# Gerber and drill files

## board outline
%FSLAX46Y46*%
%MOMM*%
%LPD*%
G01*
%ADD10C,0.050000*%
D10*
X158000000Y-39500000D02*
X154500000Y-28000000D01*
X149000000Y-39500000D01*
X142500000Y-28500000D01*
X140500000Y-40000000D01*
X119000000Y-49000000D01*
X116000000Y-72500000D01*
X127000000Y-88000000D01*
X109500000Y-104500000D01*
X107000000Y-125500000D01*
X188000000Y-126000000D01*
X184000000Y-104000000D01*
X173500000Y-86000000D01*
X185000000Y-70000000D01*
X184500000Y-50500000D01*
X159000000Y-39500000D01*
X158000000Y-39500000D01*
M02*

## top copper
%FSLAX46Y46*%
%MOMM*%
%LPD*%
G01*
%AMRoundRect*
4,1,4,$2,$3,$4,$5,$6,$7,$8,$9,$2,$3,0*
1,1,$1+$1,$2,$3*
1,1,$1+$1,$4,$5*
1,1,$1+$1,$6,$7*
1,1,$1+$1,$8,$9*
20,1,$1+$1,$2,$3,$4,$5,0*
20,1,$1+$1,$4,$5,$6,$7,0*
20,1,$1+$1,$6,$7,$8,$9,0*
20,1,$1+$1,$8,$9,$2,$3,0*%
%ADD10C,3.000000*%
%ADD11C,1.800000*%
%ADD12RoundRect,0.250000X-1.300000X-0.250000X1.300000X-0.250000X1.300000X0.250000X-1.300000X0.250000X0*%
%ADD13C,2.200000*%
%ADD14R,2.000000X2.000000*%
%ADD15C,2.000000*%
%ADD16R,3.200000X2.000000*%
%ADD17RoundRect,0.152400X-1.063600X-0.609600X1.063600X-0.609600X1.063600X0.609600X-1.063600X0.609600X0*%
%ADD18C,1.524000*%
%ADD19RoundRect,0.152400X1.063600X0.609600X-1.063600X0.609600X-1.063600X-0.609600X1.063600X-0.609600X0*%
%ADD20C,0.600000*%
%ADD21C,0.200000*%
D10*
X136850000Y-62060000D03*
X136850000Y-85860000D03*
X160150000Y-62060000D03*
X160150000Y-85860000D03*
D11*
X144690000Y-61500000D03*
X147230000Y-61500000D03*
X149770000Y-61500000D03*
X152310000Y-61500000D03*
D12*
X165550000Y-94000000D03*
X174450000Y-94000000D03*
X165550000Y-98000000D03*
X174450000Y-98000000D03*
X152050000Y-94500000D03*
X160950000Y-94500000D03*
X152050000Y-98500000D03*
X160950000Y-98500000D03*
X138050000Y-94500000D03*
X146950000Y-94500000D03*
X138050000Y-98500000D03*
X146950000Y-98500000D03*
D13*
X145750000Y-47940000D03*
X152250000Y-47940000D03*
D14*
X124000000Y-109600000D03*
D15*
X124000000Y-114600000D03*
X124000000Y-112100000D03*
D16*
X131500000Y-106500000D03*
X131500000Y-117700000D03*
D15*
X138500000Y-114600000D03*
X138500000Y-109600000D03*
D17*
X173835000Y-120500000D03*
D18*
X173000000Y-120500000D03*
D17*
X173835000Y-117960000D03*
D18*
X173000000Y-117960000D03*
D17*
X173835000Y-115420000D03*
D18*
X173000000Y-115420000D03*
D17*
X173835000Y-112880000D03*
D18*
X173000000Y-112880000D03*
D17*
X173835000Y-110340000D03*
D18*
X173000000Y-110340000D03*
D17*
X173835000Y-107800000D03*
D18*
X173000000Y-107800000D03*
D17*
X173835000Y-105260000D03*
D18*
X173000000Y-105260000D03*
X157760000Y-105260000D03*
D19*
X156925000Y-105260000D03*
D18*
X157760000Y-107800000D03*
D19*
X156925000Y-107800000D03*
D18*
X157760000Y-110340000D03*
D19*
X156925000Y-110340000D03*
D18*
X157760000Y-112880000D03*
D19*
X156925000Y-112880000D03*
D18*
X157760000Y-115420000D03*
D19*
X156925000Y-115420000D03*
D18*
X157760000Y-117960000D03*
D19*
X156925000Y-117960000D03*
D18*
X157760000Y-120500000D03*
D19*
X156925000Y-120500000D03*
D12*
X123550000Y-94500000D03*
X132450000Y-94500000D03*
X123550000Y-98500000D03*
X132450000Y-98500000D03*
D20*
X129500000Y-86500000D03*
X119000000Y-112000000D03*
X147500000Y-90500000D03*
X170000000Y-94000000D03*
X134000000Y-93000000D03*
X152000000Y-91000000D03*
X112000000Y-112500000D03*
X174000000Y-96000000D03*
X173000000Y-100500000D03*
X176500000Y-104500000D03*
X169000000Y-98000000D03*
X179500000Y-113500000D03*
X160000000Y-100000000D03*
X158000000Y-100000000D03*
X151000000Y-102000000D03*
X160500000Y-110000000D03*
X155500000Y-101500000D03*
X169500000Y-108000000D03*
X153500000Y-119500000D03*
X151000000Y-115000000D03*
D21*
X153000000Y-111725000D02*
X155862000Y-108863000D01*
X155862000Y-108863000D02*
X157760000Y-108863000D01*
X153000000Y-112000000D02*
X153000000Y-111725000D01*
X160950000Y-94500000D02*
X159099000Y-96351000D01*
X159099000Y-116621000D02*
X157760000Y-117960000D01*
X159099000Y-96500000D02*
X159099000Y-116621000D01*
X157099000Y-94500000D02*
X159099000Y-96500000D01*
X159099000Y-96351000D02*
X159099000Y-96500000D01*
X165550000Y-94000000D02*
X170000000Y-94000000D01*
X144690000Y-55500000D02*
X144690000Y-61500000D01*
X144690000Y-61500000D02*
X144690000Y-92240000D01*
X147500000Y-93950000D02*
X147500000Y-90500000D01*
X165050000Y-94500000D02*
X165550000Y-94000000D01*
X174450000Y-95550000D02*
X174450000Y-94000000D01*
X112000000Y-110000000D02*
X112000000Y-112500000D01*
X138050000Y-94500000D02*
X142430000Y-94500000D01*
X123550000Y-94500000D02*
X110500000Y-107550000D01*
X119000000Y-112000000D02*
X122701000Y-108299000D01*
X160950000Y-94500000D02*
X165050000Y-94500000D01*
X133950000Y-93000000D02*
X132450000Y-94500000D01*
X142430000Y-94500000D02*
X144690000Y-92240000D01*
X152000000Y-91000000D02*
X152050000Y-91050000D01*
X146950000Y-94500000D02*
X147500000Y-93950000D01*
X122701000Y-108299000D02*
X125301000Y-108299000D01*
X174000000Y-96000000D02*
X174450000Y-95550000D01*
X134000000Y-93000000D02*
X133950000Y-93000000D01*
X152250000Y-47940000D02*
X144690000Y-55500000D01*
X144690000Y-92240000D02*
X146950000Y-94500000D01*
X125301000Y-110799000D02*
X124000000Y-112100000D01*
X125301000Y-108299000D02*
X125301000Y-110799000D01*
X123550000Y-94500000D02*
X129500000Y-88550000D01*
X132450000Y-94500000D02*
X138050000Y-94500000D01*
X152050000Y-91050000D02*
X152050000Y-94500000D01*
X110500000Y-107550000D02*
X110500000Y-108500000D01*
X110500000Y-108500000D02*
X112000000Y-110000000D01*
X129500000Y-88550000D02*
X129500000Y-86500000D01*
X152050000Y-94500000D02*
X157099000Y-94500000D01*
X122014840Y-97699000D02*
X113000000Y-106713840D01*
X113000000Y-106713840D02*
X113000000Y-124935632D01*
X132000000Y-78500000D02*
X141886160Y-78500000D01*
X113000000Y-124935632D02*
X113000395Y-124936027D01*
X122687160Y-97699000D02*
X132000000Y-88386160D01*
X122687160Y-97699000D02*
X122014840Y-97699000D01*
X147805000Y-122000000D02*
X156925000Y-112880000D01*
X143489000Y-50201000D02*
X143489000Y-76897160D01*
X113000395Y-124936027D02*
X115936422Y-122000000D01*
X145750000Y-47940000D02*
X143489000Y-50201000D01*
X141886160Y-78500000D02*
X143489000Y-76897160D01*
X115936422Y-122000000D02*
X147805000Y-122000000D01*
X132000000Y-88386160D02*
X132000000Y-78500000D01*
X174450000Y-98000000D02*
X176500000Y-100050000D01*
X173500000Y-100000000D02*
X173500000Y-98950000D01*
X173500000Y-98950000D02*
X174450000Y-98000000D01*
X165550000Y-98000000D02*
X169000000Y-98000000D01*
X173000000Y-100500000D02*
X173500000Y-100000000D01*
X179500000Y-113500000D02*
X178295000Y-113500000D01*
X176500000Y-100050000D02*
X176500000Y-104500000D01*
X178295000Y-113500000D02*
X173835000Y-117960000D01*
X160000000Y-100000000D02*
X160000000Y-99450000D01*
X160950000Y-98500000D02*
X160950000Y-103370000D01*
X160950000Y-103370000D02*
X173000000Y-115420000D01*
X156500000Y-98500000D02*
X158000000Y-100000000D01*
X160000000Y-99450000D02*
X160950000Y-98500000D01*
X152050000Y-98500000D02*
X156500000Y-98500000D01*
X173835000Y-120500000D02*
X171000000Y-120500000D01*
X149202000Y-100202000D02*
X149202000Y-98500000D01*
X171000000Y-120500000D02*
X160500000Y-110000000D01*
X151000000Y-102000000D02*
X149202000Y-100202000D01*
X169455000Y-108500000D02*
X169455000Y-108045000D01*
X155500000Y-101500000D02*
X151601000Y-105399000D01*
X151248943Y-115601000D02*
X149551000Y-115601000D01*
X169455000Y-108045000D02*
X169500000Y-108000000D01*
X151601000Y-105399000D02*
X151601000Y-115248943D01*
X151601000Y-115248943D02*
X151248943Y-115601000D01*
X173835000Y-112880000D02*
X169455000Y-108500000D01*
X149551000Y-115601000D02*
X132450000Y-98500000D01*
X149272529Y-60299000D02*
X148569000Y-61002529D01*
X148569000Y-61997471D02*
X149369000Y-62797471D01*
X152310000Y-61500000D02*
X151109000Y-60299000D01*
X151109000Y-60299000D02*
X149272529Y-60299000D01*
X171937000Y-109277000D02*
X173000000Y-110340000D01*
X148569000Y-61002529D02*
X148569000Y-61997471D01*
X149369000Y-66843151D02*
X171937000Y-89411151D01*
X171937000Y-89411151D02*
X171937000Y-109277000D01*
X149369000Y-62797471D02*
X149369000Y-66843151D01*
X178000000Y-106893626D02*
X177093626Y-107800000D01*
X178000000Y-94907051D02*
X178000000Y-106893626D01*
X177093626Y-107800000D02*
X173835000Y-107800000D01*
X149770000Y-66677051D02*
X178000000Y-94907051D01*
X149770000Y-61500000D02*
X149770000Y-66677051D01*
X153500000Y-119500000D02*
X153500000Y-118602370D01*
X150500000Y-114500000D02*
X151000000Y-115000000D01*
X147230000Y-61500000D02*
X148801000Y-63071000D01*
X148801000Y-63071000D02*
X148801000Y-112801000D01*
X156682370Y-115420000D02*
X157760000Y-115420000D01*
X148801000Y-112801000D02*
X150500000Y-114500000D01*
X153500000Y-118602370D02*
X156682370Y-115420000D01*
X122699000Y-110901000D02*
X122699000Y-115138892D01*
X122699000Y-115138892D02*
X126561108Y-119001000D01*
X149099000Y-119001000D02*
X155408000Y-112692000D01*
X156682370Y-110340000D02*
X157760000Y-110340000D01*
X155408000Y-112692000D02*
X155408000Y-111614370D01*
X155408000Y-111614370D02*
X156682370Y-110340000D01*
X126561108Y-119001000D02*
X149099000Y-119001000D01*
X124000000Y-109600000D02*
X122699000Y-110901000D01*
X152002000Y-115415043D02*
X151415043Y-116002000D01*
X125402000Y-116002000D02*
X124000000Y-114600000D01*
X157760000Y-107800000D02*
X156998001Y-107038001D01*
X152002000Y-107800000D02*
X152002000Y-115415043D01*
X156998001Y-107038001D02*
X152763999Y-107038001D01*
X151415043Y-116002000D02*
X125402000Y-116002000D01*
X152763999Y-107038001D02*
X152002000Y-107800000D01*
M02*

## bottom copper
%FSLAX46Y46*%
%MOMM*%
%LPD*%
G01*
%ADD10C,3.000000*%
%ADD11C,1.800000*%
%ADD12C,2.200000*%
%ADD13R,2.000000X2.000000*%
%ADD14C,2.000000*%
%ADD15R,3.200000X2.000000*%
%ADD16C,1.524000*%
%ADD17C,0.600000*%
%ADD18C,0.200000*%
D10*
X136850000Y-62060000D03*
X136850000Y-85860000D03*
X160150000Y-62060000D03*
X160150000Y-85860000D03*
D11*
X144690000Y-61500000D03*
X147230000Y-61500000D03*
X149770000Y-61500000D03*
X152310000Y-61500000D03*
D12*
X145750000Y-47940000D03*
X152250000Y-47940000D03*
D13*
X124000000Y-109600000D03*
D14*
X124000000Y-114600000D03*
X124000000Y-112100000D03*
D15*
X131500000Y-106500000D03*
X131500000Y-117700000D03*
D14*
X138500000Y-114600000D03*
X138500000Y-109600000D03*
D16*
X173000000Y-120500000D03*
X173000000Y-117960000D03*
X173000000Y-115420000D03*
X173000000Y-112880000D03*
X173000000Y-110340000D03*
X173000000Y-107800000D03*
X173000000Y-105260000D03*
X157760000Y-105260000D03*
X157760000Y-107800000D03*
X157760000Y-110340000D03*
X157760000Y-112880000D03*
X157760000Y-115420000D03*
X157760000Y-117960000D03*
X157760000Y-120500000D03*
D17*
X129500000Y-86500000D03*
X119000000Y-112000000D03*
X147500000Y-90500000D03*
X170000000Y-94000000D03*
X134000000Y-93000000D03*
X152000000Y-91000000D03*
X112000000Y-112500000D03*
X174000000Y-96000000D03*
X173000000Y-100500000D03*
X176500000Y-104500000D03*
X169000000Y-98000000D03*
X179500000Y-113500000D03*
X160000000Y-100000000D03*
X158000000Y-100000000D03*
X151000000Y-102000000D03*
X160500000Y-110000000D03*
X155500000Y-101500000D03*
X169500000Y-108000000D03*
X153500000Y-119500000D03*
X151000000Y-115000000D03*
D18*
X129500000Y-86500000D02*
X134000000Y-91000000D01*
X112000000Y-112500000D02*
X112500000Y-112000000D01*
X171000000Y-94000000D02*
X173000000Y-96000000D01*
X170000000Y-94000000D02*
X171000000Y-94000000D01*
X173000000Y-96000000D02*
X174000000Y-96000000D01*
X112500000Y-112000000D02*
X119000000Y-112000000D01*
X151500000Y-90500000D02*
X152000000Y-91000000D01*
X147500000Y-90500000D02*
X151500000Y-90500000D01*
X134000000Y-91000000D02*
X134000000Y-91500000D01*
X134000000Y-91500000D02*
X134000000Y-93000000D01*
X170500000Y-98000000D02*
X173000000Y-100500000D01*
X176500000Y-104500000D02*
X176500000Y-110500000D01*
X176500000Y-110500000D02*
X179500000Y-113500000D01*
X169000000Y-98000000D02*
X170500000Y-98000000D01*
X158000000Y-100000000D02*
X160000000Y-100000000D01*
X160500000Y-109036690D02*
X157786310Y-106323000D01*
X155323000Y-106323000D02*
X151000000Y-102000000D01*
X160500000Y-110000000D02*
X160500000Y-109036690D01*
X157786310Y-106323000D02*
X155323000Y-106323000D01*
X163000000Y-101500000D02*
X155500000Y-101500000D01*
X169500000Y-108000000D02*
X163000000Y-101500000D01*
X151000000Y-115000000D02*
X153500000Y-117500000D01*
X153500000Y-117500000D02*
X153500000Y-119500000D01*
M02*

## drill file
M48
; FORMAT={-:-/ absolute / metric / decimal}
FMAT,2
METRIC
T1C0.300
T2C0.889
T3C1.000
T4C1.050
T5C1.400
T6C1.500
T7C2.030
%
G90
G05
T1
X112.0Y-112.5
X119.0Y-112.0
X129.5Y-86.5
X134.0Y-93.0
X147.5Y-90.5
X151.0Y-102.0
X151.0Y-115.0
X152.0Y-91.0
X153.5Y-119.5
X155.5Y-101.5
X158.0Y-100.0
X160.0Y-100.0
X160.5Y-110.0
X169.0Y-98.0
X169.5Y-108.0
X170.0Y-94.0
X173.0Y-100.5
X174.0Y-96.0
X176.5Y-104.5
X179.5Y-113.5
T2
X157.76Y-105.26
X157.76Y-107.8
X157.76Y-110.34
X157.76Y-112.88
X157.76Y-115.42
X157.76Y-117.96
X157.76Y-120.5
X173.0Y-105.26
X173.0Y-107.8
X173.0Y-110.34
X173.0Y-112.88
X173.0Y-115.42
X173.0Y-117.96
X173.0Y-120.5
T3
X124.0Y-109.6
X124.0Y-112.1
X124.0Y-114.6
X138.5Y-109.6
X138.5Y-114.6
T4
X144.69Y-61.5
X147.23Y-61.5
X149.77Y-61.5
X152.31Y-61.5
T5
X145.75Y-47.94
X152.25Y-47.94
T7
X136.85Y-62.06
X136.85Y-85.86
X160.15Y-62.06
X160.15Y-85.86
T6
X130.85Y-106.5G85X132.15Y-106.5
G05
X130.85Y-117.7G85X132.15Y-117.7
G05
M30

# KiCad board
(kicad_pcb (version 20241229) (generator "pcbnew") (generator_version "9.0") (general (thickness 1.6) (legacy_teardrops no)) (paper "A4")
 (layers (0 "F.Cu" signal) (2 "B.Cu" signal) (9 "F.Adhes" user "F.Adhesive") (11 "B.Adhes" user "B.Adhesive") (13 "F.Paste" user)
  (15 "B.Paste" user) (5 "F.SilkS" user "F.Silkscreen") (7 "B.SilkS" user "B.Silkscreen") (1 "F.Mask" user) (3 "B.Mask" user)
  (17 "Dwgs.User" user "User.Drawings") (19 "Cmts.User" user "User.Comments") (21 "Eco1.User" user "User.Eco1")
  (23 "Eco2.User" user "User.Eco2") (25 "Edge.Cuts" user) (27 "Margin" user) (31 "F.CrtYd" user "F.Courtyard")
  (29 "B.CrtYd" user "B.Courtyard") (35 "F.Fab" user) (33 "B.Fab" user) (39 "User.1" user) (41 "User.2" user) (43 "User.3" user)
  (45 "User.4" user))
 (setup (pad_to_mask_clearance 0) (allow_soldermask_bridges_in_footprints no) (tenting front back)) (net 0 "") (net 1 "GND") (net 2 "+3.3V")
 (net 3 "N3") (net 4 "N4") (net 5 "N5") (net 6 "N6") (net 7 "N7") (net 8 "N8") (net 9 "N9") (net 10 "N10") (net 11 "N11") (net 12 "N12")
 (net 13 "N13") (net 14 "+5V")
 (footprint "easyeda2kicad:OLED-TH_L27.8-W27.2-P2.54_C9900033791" (layer "F.Cu") (at 148.5 61.5)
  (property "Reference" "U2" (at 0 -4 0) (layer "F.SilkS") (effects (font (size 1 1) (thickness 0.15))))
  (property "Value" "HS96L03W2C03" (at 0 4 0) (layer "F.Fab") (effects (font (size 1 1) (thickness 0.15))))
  (pad "" thru_hole circle (at -11.65 0.56) (size 3 3) (drill 2.03) (layers "*.Cu" "*.Mask") (remove_unused_layers no))
  (pad "" thru_hole circle (at -11.65 24.36) (size 3 3) (drill 2.03) (layers "*.Cu" "*.Mask") (remove_unused_layers no))
  (pad "" thru_hole circle (at 11.65 0.56) (size 3 3) (drill 2.03) (layers "*.Cu" "*.Mask") (remove_unused_layers no))
  (pad "" thru_hole circle (at 11.65 24.36) (size 3 3) (drill 2.03) (layers "*.Cu" "*.Mask") (remove_unused_layers no))
  (pad "1" thru_hole circle (at -3.81 0) (size 1.8 1.8) (drill 1.049986) (layers "*.Cu" "*.Mask") (remove_unused_layers no) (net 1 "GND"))
  (pad "2" thru_hole circle (at -1.27 0) (size 1.8 1.8) (drill 1.049986) (layers "*.Cu" "*.Mask") (remove_unused_layers no) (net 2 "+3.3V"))
  (pad "3" thru_hole circle (at 1.27 0) (size 1.8 1.8) (drill 1.049986) (layers "*.Cu" "*.Mask") (remove_unused_layers no) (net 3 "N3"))
  (pad "4" thru_hole circle (at 3.81 0) (size 1.8 1.8) (drill 1.049986) (layers "*.Cu" "*.Mask") (remove_unused_layers no) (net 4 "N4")))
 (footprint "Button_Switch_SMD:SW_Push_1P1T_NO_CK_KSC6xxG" (layer "F.Cu") (at 170 96)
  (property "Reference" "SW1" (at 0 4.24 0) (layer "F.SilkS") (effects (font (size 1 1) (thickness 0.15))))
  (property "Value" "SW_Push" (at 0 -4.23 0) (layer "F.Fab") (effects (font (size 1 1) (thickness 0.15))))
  (pad "1" smd roundrect (at -4.45 -2) (size 3.1 1) (layers "F.Cu" "F.Mask" "F.Paste") (roundrect_rratio 0.25) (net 1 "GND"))
  (pad "1" smd roundrect (at 4.45 -2) (size 3.1 1) (layers "F.Cu" "F.Mask" "F.Paste") (roundrect_rratio 0.25) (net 1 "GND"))
  (pad "2" smd roundrect (at -4.45 2) (size 3.1 1) (layers "F.Cu" "F.Mask" "F.Paste") (roundrect_rratio 0.25) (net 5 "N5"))
  (pad "2" smd roundrect (at 4.45 2) (size 3.1 1) (layers "F.Cu" "F.Mask" "F.Paste") (roundrect_rratio 0.25) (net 5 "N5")))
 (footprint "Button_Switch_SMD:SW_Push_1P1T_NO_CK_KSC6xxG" (layer "F.Cu") (at 156.5 96.5)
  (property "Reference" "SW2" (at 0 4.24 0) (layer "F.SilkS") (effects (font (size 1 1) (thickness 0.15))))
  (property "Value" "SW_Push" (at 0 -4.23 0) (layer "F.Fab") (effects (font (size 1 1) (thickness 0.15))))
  (pad "1" smd roundrect (at -4.45 -2) (size 3.1 1) (layers "F.Cu" "F.Mask" "F.Paste") (roundrect_rratio 0.25) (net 1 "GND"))
  (pad "1" smd roundrect (at 4.45 -2) (size 3.1 1) (layers "F.Cu" "F.Mask" "F.Paste") (roundrect_rratio 0.25) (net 1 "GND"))
  (pad "2" smd roundrect (at -4.45 2) (size 3.1 1) (layers "F.Cu" "F.Mask" "F.Paste") (roundrect_rratio 0.25) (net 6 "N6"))
  (pad "2" smd roundrect (at 4.45 2) (size 3.1 1) (layers "F.Cu" "F.Mask" "F.Paste") (roundrect_rratio 0.25) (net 6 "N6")))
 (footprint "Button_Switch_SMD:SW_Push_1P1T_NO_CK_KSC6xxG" (layer "F.Cu") (at 142.5 96.5)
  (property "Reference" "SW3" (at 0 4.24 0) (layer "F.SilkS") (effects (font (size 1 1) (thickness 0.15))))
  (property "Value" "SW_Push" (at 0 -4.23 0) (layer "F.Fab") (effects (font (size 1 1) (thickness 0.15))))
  (pad "1" smd roundrect (at -4.45 -2) (size 3.1 1) (layers "F.Cu" "F.Mask" "F.Paste") (roundrect_rratio 0.25) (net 1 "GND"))
  (pad "1" smd roundrect (at 4.45 -2) (size 3.1 1) (layers "F.Cu" "F.Mask" "F.Paste") (roundrect_rratio 0.25) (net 1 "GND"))
  (pad "2" smd roundrect (at -4.45 2) (size 3.1 1) (layers "F.Cu" "F.Mask" "F.Paste") (roundrect_rratio 0.25) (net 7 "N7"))
  (pad "2" smd roundrect (at 4.45 2) (size 3.1 1) (layers "F.Cu" "F.Mask" "F.Paste") (roundrect_rratio 0.25) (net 7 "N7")))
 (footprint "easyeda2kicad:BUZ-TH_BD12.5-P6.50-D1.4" (layer "F.Cu") (at 149 47.94)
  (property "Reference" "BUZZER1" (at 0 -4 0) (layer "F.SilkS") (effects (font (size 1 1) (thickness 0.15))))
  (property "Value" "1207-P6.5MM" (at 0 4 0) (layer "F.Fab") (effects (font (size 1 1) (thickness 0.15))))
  (pad "1" thru_hole circle (at -3.25 0) (size 2.2 2.2) (drill 1.399998) (layers "*.Cu" "*.Mask") (remove_unused_layers no) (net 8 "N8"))
  (pad "2" thru_hole circle (at 3.25 0) (size 2.2 2.2) (drill 1.399998) (layers "*.Cu" "*.Mask") (remove_unused_layers no) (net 1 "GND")))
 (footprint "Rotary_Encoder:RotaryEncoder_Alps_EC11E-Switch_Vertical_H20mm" (layer "F.Cu") (at 124 109.6)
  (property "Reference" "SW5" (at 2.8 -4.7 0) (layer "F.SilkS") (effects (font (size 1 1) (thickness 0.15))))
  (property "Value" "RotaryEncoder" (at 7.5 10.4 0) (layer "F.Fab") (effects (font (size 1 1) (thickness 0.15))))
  (pad "A" thru_hole rect (at 0 0) (size 2 2) (drill 1) (layers "*.Cu" "*.Mask") (remove_unused_layers no) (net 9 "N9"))
  (pad "B" thru_hole circle (at 0 5) (size 2 2) (drill 1) (layers "*.Cu" "*.Mask") (remove_unused_layers no) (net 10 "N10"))
  (pad "C" thru_hole circle (at 0 2.5) (size 2 2) (drill 1) (layers "*.Cu" "*.Mask") (remove_unused_layers no) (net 1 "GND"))
  (pad "MP" thru_hole rect (at 7.5 -3.1) (size 3.2 2) (drill oval 2.8 1.5) (layers "*.Cu" "*.Mask") (remove_unused_layers no))
  (pad "MP" thru_hole rect (at 7.5 8.1) (size 3.2 2) (drill oval 2.8 1.5) (layers "*.Cu" "*.Mask") (remove_unused_layers no))
  (pad "S1" thru_hole circle (at 14.5 5) (size 2 2) (drill 1) (layers "*.Cu" "*.Mask") (remove_unused_layers no))
  (pad "S2" thru_hole circle (at 14.5 0) (size 2 2) (drill 1) (layers "*.Cu" "*.Mask") (remove_unused_layers no)))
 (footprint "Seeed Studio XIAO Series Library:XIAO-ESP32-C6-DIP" (layer "F.Cu") (at 165.38 112.88 -90)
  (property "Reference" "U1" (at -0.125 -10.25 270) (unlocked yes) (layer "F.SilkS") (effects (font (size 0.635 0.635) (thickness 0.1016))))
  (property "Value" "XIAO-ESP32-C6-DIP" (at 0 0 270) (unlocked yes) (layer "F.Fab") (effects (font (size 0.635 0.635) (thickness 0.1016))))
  (pad "1" smd roundrect (at 7.62 -8.455) (size 2.432 1.524) (layers "F.Cu" "F.Mask") (roundrect_rratio 0.1) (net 7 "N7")
   (thermal_bridge_angle 45))
  (pad "1" thru_hole circle (at 7.62 -7.62) (size 1.524 1.524) (drill 0.889) (layers "*.Cu" "*.Mask") (remove_unused_layers no) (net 7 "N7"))
  (pad "2" smd roundrect (at 5.08 -8.455) (size 2.432 1.524) (layers "F.Cu" "F.Mask") (roundrect_rratio 0.1) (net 5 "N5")
   (thermal_bridge_angle 45))
  (pad "2" thru_hole circle (at 5.08 -7.62) (size 1.524 1.524) (drill 0.889) (layers "*.Cu" "*.Mask") (remove_unused_layers no) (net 5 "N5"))
  (pad "3" smd roundrect (at 2.54 -8.455) (size 2.432 1.524) (layers "F.Cu" "F.Mask") (roundrect_rratio 0.1) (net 6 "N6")
   (thermal_bridge_angle 45))
  (pad "3" thru_hole circle (at 2.54 -7.62) (size 1.524 1.524) (drill 0.889) (layers "*.Cu" "*.Mask") (remove_unused_layers no) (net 6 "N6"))
  (pad "4" smd roundrect (at 0 -8.455) (size 2.432 1.524) (layers "F.Cu" "F.Mask") (roundrect_rratio 0.1) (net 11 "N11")
   (thermal_bridge_angle 45))
  (pad "4" thru_hole circle (at 0 -7.62) (size 1.524 1.524) (drill 0.889) (layers "*.Cu" "*.Mask") (remove_unused_layers no) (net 11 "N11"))
  (pad "5" smd roundrect (at -2.54 -8.455) (size 2.432 1.524) (layers "F.Cu" "F.Mask") (roundrect_rratio 0.1) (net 4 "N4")
   (thermal_bridge_angle 45))
  (pad "5" thru_hole circle (at -2.54 -7.62) (size 1.524 1.524) (drill 0.889) (layers "*.Cu" "*.Mask") (remove_unused_layers no)
   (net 4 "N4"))
  (pad "6" smd roundrect (at -5.08 -8.455) (size 2.432 1.524) (layers "F.Cu" "F.Mask") (roundrect_rratio 0.1) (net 3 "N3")
   (thermal_bridge_angle 45))
  (pad "6" thru_hole circle (at -5.08 -7.62) (size 1.524 1.524) (drill 0.889) (layers "*.Cu" "*.Mask") (remove_unused_layers no)
   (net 3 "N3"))
  (pad "7" smd roundrect (at -7.62 -8.455) (size 2.432 1.524) (layers "F.Cu" "F.Mask") (roundrect_rratio 0.1) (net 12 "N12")
   (thermal_bridge_angle 45))
  (pad "7" thru_hole circle (at -7.62 -7.62) (size 1.524 1.524) (drill 0.889) (layers "*.Cu" "*.Mask") (remove_unused_layers no)
   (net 12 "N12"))
  (pad "8" thru_hole circle (at -7.62 7.62 180) (size 1.524 1.524) (drill 0.889) (layers "*.Cu" "*.Mask") (remove_unused_layers no)
   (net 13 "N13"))
  (pad "8" smd roundrect (at -7.62 8.455 180) (size 2.432 1.524) (layers "F.Cu" "F.Mask") (roundrect_rratio 0.1) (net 13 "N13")
   (thermal_bridge_angle 45))
  (pad "9" thru_hole circle (at -5.08 7.62 180) (size 1.524 1.524) (drill 0.889) (layers "*.Cu" "*.Mask") (remove_unused_layers no)
   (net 10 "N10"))
  (pad "9" smd roundrect (at -5.08 8.455 180) (size 2.432 1.524) (layers "F.Cu" "F.Mask") (roundrect_rratio 0.1) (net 10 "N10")
   (thermal_bridge_angle 45))
  (pad "10" thru_hole circle (at -2.54 7.62 180) (size 1.524 1.524) (drill 0.889) (layers "*.Cu" "*.Mask") (remove_unused_layers no)
   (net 9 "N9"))
  (pad "10" smd roundrect (at -2.54 8.455 180) (size 2.432 1.524) (layers "F.Cu" "F.Mask") (roundrect_rratio 0.1) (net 9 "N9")
   (thermal_bridge_angle 45))
  (pad "11" thru_hole circle (at 0 7.62 180) (size 1.524 1.524) (drill 0.889) (layers "*.Cu" "*.Mask") (remove_unused_layers no)
   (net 8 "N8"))
  (pad "11" smd roundrect (at 0 8.455 180) (size 2.432 1.524) (layers "F.Cu" "F.Mask") (roundrect_rratio 0.1) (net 8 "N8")
   (thermal_bridge_angle 45))
  (pad "12" thru_hole circle (at 2.54 7.62 180) (size 1.524 1.524) (drill 0.889) (layers "*.Cu" "*.Mask") (remove_unused_layers no)
   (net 2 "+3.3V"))
  (pad "12" smd roundrect (at 2.54 8.455 180) (size 2.432 1.524) (layers "F.Cu" "F.Mask") (roundrect_rratio 0.1) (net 2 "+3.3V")
   (thermal_bridge_angle 45))
  (pad "13" thru_hole circle (at 5.08 7.62 180) (size 1.524 1.524) (drill 0.889) (layers "*.Cu" "*.Mask") (remove_unused_layers no)
   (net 1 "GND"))
  (pad "13" smd roundrect (at 5.08 8.455 180) (size 2.432 1.524) (layers "F.Cu" "F.Mask") (roundrect_rratio 0.1) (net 1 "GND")
   (thermal_bridge_angle 45))
  (pad "14" thru_hole circle (at 7.62 7.62 180) (size 1.524 1.524) (drill 0.889) (layers "*.Cu" "*.Mask") (remove_unused_layers no)
   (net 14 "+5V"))
  (pad "14" smd roundrect (at 7.62 8.455 180) (size 2.432 1.524) (layers "F.Cu" "F.Mask") (roundrect_rratio 0.1) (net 14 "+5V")
   (thermal_bridge_angle 45)))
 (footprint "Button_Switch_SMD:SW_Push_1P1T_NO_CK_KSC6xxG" (layer "F.Cu") (at 128 96.5)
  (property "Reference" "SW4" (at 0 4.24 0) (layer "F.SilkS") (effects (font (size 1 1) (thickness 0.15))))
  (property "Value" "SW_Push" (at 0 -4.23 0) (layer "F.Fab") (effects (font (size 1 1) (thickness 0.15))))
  (pad "1" smd roundrect (at -4.45 -2) (size 3.1 1) (layers "F.Cu" "F.Mask" "F.Paste") (roundrect_rratio 0.25) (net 1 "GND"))
  (pad "1" smd roundrect (at 4.45 -2) (size 3.1 1) (layers "F.Cu" "F.Mask" "F.Paste") (roundrect_rratio 0.25) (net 1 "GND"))
  (pad "2" smd roundrect (at -4.45 2) (size 3.1 1) (layers "F.Cu" "F.Mask" "F.Paste") (roundrect_rratio 0.25) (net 11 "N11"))
  (pad "2" smd roundrect (at 4.45 2) (size 3.1 1) (layers "F.Cu" "F.Mask" "F.Paste") (roundrect_rratio 0.25) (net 11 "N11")))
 (gr_poly
  (pts (xy 158 39.5) (xy 154.5 28) (xy 149 39.5) (xy 142.5 28.5) (xy 140.5 40) (xy 119 49) (xy 116 72.5) (xy 127 88) (xy 109.5 104.5)
   (xy 107 125.5) (xy 188 126) (xy 184 104) (xy 173.5 86) (xy 185 70) (xy 184.5 50.5) (xy 159 39.5))
  (stroke (width 0.05) (type solid)) (fill no) (layer "Edge.Cuts"))
 (segment (start 153 111.725) (end 155.862 108.863) (width 0.2) (layer "F.Cu") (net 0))
 (segment (start 155.862 108.863) (end 157.76 108.863) (width 0.2) (layer "F.Cu") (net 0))
 (segment (start 153 112) (end 153 111.725) (width 0.2) (layer "F.Cu") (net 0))
 (segment (start 160.95 94.5) (end 159.099 96.351) (width 0.2) (layer "F.Cu") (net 1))
 (segment (start 159.099 116.621) (end 157.76 117.96) (width 0.2) (layer "F.Cu") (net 1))
 (segment (start 159.099 96.5) (end 159.099 116.621) (width 0.2) (layer "F.Cu") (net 1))
 (segment (start 157.099 94.5) (end 159.099 96.5) (width 0.2) (layer "F.Cu") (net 1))
 (segment (start 159.099 96.351) (end 159.099 96.5) (width 0.2) (layer "F.Cu") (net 1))
 (segment (start 165.55 94) (end 170 94) (width 0.2) (layer "F.Cu") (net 1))
 (segment (start 144.69 55.5) (end 144.69 61.5) (width 0.2) (layer "F.Cu") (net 1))
 (segment (start 144.69 61.5) (end 144.69 92.24) (width 0.2) (layer "F.Cu") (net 1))
 (segment (start 147.5 93.95) (end 147.5 90.5) (width 0.2) (layer "F.Cu") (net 1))
 (segment (start 165.05 94.5) (end 165.55 94) (width 0.2) (layer "F.Cu") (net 1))
 (segment (start 174.45 95.55) (end 174.45 94) (width 0.2) (layer "F.Cu") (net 1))
 (segment (start 112 110) (end 112 112.5) (width 0.2) (layer "F.Cu") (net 1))
 (segment (start 138.05 94.5) (end 142.43 94.5) (width 0.2) (layer "F.Cu") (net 1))
 (segment (start 123.55 94.5) (end 110.5 107.55) (width 0.2) (layer "F.Cu") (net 1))
 (segment (start 119 112) (end 122.701 108.299) (width 0.2) (layer "F.Cu") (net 1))
 (segment (start 160.95 94.5) (end 165.05 94.5) (width 0.2) (layer "F.Cu") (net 1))
 (segment (start 133.95 93) (end 132.45 94.5) (width 0.2) (layer "F.Cu") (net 1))
 (segment (start 142.43 94.5) (end 144.69 92.24) (width 0.2) (layer "F.Cu") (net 1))
 (segment (start 152 91) (end 152.05 91.05) (width 0.2) (layer "F.Cu") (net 1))
 (segment (start 146.95 94.5) (end 147.5 93.95) (width 0.2) (layer "F.Cu") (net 1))
 (segment (start 122.701 108.299) (end 125.301 108.299) (width 0.2) (layer "F.Cu") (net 1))
 (segment (start 174 96) (end 174.45 95.55) (width 0.2) (layer "F.Cu") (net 1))
 (segment (start 134 93) (end 133.95 93) (width 0.2) (layer "F.Cu") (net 1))
 (segment (start 152.25 47.94) (end 144.69 55.5) (width 0.2) (layer "F.Cu") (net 1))
 (segment (start 144.69 92.24) (end 146.95 94.5) (width 0.2) (layer "F.Cu") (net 1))
 (segment (start 125.301 110.799) (end 124 112.1) (width 0.2) (layer "F.Cu") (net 1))
 (segment (start 125.301 108.299) (end 125.301 110.799) (width 0.2) (layer "F.Cu") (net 1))
 (segment (start 123.55 94.5) (end 129.5 88.55) (width 0.2) (layer "F.Cu") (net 1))
 (segment (start 132.45 94.5) (end 138.05 94.5) (width 0.2) (layer "F.Cu") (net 1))
 (segment (start 152.05 91.05) (end 152.05 94.5) (width 0.2) (layer "F.Cu") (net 1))
 (segment (start 110.5 107.55) (end 110.5 108.5) (width 0.2) (layer "F.Cu") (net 1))
 (segment (start 110.5 108.5) (end 112 110) (width 0.2) (layer "F.Cu") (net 1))
 (segment (start 129.5 88.55) (end 129.5 86.5) (width 0.2) (layer "F.Cu") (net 1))
 (segment (start 152.05 94.5) (end 157.099 94.5) (width 0.2) (layer "F.Cu") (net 1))
 (via (at 129.5 86.5) (size 0.6) (drill 0.3) (layers "F.Cu" "B.Cu") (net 1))
 (via (at 119 112) (size 0.6) (drill 0.3) (layers "F.Cu" "B.Cu") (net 1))
 (via (at 147.5 90.5) (size 0.6) (drill 0.3) (layers "F.Cu" "B.Cu") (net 1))
 (via (at 170 94) (size 0.6) (drill 0.3) (layers "F.Cu" "B.Cu") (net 1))
 (via (at 134 93) (size 0.6) (drill 0.3) (layers "F.Cu" "B.Cu") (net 1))
 (via (at 152 91) (size 0.6) (drill 0.3) (layers "F.Cu" "B.Cu") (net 1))
 (via (at 112 112.5) (size 0.6) (drill 0.3) (layers "F.Cu" "B.Cu") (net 1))
 (via (at 174 96) (size 0.6) (drill 0.3) (layers "F.Cu" "B.Cu") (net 1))
 (segment (start 129.5 86.5) (end 134 91) (width 0.2) (layer "B.Cu") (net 1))
 (segment (start 112 112.5) (end 112.5 112) (width 0.2) (layer "B.Cu") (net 1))
 (segment (start 171 94) (end 173 96) (width 0.2) (layer "B.Cu") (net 1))
 (segment (start 170 94) (end 171 94) (width 0.2) (layer "B.Cu") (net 1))
 (segment (start 173 96) (end 174 96) (width 0.2) (layer "B.Cu") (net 1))
 (segment (start 112.5 112) (end 119 112) (width 0.2) (layer "B.Cu") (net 1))
 (segment (start 151.5 90.5) (end 152 91) (width 0.2) (layer "B.Cu") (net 1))
 (segment (start 147.5 90.5) (end 151.5 90.5) (width 0.2) (layer "B.Cu") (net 1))
 (segment (start 134 91) (end 134 91.5) (width 0.2) (layer "B.Cu") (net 1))
 (segment (start 134 91.5) (end 134 93) (width 0.2) (layer "B.Cu") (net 1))
 (segment (start 122.01484 97.699) (end 113 106.71384) (width 0.2) (layer "F.Cu") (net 8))
 (segment (start 113 106.71384) (end 113 124.935632) (width 0.2) (layer "F.Cu") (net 8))
 (segment (start 132 78.5) (end 141.88616 78.5) (width 0.2) (layer "F.Cu") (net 8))
 (segment (start 113 124.935632) (end 113.000395 124.936027) (width 0.2) (layer "F.Cu") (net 8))
 (segment (start 122.68716 97.699) (end 132 88.38616) (width 0.2) (layer "F.Cu") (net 8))
 (segment (start 122.68716 97.699) (end 122.01484 97.699) (width 0.2) (layer "F.Cu") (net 8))
 (segment (start 147.805 122) (end 156.925 112.88) (width 0.2) (layer "F.Cu") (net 8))
 (segment (start 143.489 50.201) (end 143.489 76.89716) (width 0.2) (layer "F.Cu") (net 8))
 (segment (start 113.000395 124.936027) (end 115.936422 122) (width 0.2) (layer "F.Cu") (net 8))
 (segment (start 145.75 47.94) (end 143.489 50.201) (width 0.2) (layer "F.Cu") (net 8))
 (segment (start 141.88616 78.5) (end 143.489 76.89716) (width 0.2) (layer "F.Cu") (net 8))
 (segment (start 115.936422 122) (end 147.805 122) (width 0.2) (layer "F.Cu") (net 8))
 (segment (start 132 88.38616) (end 132 78.5) (width 0.2) (layer "F.Cu") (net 8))
 (segment (start 174.45 98) (end 176.5 100.05) (width 0.2) (layer "F.Cu") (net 5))
 (segment (start 173.5 100) (end 173.5 98.95) (width 0.2) (layer "F.Cu") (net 5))
 (segment (start 173.5 98.95) (end 174.45 98) (width 0.2) (layer "F.Cu") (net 5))
 (segment (start 165.55 98) (end 169 98) (width 0.2) (layer "F.Cu") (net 5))
 (segment (start 173 100.5) (end 173.5 100) (width 0.2) (layer "F.Cu") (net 5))
 (segment (start 179.5 113.5) (end 178.295 113.5) (width 0.2) (layer "F.Cu") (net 5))
 (segment (start 176.5 100.05) (end 176.5 104.5) (width 0.2) (layer "F.Cu") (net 5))
 (segment (start 178.295 113.5) (end 173.835 117.96) (width 0.2) (layer "F.Cu") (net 5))
 (via (at 173 100.5) (size 0.6) (drill 0.3) (layers "F.Cu" "B.Cu") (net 5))
 (via (at 176.5 104.5) (size 0.6) (drill 0.3) (layers "F.Cu" "B.Cu") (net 5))
 (via (at 169 98) (size 0.6) (drill 0.3) (layers "F.Cu" "B.Cu") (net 5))
 (via (at 179.5 113.5) (size 0.6) (drill 0.3) (layers "F.Cu" "B.Cu") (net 5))
 (segment (start 170.5 98) (end 173 100.5) (width 0.2) (layer "B.Cu") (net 5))
 (segment (start 176.5 104.5) (end 176.5 110.5) (width 0.2) (layer "B.Cu") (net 5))
 (segment (start 176.5 110.5) (end 179.5 113.5) (width 0.2) (layer "B.Cu") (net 5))
 (segment (start 169 98) (end 170.5 98) (width 0.2) (layer "B.Cu") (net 5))
 (segment (start 160 100) (end 160 99.45) (width 0.2) (layer "F.Cu") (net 6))
 (segment (start 160.95 98.5) (end 160.95 103.37) (width 0.2) (layer "F.Cu") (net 6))
 (segment (start 160.95 103.37) (end 173 115.42) (width 0.2) (layer "F.Cu") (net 6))
 (segment (start 156.5 98.5) (end 158 100) (width 0.2) (layer "F.Cu") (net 6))
 (segment (start 160 99.45) (end 160.95 98.5) (width 0.2) (layer "F.Cu") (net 6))
 (segment (start 152.05 98.5) (end 156.5 98.5) (width 0.2) (layer "F.Cu") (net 6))
 (via (at 160 100) (size 0.6) (drill 0.3) (layers "F.Cu" "B.Cu") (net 6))
 (via (at 158 100) (size 0.6) (drill 0.3) (layers "F.Cu" "B.Cu") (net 6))
 (segment (start 158 100) (end 160 100) (width 0.2) (layer "B.Cu") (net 6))
 (segment (start 173.835 120.5) (end 171 120.5) (width 0.2) (layer "F.Cu") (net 7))
 (segment (start 149.202 100.202) (end 149.202 98.5) (width 0.2) (layer "F.Cu") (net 7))
 (segment (start 171 120.5) (end 160.5 110) (width 0.2) (layer "F.Cu") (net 7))
 (segment (start 151 102) (end 149.202 100.202) (width 0.2) (layer "F.Cu") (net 7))
 (via (at 151 102) (size 0.6) (drill 0.3) (layers "F.Cu" "B.Cu") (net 7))
 (via (at 160.5 110) (size 0.6) (drill 0.3) (layers "F.Cu" "B.Cu") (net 7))
 (segment (start 160.5 109.03669) (end 157.78631 106.323) (width 0.2) (layer "B.Cu") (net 7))
 (segment (start 155.323 106.323) (end 151 102) (width 0.2) (layer "B.Cu") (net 7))
 (segment (start 160.5 110) (end 160.5 109.03669) (width 0.2) (layer "B.Cu") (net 7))
 (segment (start 157.78631 106.323) (end 155.323 106.323) (width 0.2) (layer "B.Cu") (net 7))
 (segment (start 169.455 108.5) (end 169.455 108.045) (width 0.2) (layer "F.Cu") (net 11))
 (segment (start 155.5 101.5) (end 151.601 105.399) (width 0.2) (layer "F.Cu") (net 11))
 (segment (start 151.248943 115.601) (end 149.551 115.601) (width 0.2) (layer "F.Cu") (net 11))
 (segment (start 169.455 108.045) (end 169.5 108) (width 0.2) (layer "F.Cu") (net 11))
 (segment (start 151.601 105.399) (end 151.601 115.248943) (width 0.2) (layer "F.Cu") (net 11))
 (segment (start 151.601 115.248943) (end 151.248943 115.601) (width 0.2) (layer "F.Cu") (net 11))
 (segment (start 173.835 112.88) (end 169.455 108.5) (width 0.2) (layer "F.Cu") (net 11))
 (segment (start 149.551 115.601) (end 132.45 98.5) (width 0.2) (layer "F.Cu") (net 11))
 (via (at 155.5 101.5) (size 0.6) (drill 0.3) (layers "F.Cu" "B.Cu") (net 11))
 (via (at 169.5 108) (size 0.6) (drill 0.3) (layers "F.Cu" "B.Cu") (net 11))
 (segment (start 163 101.5) (end 155.5 101.5) (width 0.2) (layer "B.Cu") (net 11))
 (segment (start 169.5 108) (end 163 101.5) (width 0.2) (layer "B.Cu") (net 11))
 (segment (start 149.272529 60.299) (end 148.569 61.002529) (width 0.2) (layer "F.Cu") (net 4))
 (segment (start 148.569 61.997471) (end 149.369 62.797471) (width 0.2) (layer "F.Cu") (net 4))
 (segment (start 152.31 61.5) (end 151.109 60.299) (width 0.2) (layer "F.Cu") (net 4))
 (segment (start 151.109 60.299) (end 149.272529 60.299) (width 0.2) (layer "F.Cu") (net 4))
 (segment (start 171.937 109.277) (end 173 110.34) (width 0.2) (layer "F.Cu") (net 4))
 (segment (start 148.569 61.002529) (end 148.569 61.997471) (width 0.2) (layer "F.Cu") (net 4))
 (segment (start 149.369 66.843151) (end 171.937 89.411151) (width 0.2) (layer "F.Cu") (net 4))
 (segment (start 171.937 89.411151) (end 171.937 109.277) (width 0.2) (layer "F.Cu") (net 4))
 (segment (start 149.369 62.797471) (end 149.369 66.843151) (width 0.2) (layer "F.Cu") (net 4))
 (segment (start 178 106.893626) (end 177.093626 107.8) (width 0.2) (layer "F.Cu") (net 3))
 (segment (start 178 94.907051) (end 178 106.893626) (width 0.2) (layer "F.Cu") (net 3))
 (segment (start 177.093626 107.8) (end 173.835 107.8) (width 0.2) (layer "F.Cu") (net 3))
 (segment (start 149.77 66.677051) (end 178 94.907051) (width 0.2) (layer "F.Cu") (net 3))
 (segment (start 149.77 61.5) (end 149.77 66.677051) (width 0.2) (layer "F.Cu") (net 3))
 (segment (start 153.5 119.5) (end 153.5 118.60237) (width 0.2) (layer "F.Cu") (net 2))
 (segment (start 150.5 114.5) (end 151 115) (width 0.2) (layer "F.Cu") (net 2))
 (segment (start 147.23 61.5) (end 148.801 63.071) (width 0.2) (layer "F.Cu") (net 2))
 (segment (start 148.801 63.071) (end 148.801 112.801) (width 0.2) (layer "F.Cu") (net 2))
 (segment (start 156.68237 115.42) (end 157.76 115.42) (width 0.2) (layer "F.Cu") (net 2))
 (segment (start 148.801 112.801) (end 150.5 114.5) (width 0.2) (layer "F.Cu") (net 2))
 (segment (start 153.5 118.60237) (end 156.68237 115.42) (width 0.2) (layer "F.Cu") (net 2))
 (via (at 153.5 119.5) (size 0.6) (drill 0.3) (layers "F.Cu" "B.Cu") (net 2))
 (via (at 151 115) (size 0.6) (drill 0.3) (layers "F.Cu" "B.Cu") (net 2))
 (segment (start 151 115) (end 153.5 117.5) (width 0.2) (layer "B.Cu") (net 2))
 (segment (start 153.5 117.5) (end 153.5 119.5) (width 0.2) (layer "B.Cu") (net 2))
 (segment (start 122.699 110.901) (end 122.699 115.138892) (width 0.2) (layer "F.Cu") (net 9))
 (segment (start 122.699 115.138892) (end 126.561108 119.001) (width 0.2) (layer "F.Cu") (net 9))
 (segment (start 149.099 119.001) (end 155.408 112.692) (width 0.2) (layer "F.Cu") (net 9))
 (segment (start 156.68237 110.34) (end 157.76 110.34) (width 0.2) (layer "F.Cu") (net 9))
 (segment (start 155.408 112.692) (end 155.408 111.61437) (width 0.2) (layer "F.Cu") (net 9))
 (segment (start 155.408 111.61437) (end 156.68237 110.34) (width 0.2) (layer "F.Cu") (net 9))
 (segment (start 126.561108 119.001) (end 149.099 119.001) (width 0.2) (layer "F.Cu") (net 9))
 (segment (start 124 109.6) (end 122.699 110.901) (width 0.2) (layer "F.Cu") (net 9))
 (segment (start 152.002 115.415043) (end 151.415043 116.002) (width 0.2) (layer "F.Cu") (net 10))
 (segment (start 125.402 116.002) (end 124 114.6) (width 0.2) (layer "F.Cu") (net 10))
 (segment (start 157.76 107.8) (end 156.998001 107.038001) (width 0.2) (layer "F.Cu") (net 10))
 (segment (start 152.002 107.8) (end 152.002 115.415043) (width 0.2) (layer "F.Cu") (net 10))
 (segment (start 156.998001 107.038001) (end 152.763999 107.038001) (width 0.2) (layer "F.Cu") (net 10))
 (segment (start 151.415043 116.002) (end 125.402 116.002) (width 0.2) (layer "F.Cu") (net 10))
 (segment (start 152.763999 107.038001) (end 152.002 107.8) (width 0.2) (layer "F.Cu") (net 10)))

